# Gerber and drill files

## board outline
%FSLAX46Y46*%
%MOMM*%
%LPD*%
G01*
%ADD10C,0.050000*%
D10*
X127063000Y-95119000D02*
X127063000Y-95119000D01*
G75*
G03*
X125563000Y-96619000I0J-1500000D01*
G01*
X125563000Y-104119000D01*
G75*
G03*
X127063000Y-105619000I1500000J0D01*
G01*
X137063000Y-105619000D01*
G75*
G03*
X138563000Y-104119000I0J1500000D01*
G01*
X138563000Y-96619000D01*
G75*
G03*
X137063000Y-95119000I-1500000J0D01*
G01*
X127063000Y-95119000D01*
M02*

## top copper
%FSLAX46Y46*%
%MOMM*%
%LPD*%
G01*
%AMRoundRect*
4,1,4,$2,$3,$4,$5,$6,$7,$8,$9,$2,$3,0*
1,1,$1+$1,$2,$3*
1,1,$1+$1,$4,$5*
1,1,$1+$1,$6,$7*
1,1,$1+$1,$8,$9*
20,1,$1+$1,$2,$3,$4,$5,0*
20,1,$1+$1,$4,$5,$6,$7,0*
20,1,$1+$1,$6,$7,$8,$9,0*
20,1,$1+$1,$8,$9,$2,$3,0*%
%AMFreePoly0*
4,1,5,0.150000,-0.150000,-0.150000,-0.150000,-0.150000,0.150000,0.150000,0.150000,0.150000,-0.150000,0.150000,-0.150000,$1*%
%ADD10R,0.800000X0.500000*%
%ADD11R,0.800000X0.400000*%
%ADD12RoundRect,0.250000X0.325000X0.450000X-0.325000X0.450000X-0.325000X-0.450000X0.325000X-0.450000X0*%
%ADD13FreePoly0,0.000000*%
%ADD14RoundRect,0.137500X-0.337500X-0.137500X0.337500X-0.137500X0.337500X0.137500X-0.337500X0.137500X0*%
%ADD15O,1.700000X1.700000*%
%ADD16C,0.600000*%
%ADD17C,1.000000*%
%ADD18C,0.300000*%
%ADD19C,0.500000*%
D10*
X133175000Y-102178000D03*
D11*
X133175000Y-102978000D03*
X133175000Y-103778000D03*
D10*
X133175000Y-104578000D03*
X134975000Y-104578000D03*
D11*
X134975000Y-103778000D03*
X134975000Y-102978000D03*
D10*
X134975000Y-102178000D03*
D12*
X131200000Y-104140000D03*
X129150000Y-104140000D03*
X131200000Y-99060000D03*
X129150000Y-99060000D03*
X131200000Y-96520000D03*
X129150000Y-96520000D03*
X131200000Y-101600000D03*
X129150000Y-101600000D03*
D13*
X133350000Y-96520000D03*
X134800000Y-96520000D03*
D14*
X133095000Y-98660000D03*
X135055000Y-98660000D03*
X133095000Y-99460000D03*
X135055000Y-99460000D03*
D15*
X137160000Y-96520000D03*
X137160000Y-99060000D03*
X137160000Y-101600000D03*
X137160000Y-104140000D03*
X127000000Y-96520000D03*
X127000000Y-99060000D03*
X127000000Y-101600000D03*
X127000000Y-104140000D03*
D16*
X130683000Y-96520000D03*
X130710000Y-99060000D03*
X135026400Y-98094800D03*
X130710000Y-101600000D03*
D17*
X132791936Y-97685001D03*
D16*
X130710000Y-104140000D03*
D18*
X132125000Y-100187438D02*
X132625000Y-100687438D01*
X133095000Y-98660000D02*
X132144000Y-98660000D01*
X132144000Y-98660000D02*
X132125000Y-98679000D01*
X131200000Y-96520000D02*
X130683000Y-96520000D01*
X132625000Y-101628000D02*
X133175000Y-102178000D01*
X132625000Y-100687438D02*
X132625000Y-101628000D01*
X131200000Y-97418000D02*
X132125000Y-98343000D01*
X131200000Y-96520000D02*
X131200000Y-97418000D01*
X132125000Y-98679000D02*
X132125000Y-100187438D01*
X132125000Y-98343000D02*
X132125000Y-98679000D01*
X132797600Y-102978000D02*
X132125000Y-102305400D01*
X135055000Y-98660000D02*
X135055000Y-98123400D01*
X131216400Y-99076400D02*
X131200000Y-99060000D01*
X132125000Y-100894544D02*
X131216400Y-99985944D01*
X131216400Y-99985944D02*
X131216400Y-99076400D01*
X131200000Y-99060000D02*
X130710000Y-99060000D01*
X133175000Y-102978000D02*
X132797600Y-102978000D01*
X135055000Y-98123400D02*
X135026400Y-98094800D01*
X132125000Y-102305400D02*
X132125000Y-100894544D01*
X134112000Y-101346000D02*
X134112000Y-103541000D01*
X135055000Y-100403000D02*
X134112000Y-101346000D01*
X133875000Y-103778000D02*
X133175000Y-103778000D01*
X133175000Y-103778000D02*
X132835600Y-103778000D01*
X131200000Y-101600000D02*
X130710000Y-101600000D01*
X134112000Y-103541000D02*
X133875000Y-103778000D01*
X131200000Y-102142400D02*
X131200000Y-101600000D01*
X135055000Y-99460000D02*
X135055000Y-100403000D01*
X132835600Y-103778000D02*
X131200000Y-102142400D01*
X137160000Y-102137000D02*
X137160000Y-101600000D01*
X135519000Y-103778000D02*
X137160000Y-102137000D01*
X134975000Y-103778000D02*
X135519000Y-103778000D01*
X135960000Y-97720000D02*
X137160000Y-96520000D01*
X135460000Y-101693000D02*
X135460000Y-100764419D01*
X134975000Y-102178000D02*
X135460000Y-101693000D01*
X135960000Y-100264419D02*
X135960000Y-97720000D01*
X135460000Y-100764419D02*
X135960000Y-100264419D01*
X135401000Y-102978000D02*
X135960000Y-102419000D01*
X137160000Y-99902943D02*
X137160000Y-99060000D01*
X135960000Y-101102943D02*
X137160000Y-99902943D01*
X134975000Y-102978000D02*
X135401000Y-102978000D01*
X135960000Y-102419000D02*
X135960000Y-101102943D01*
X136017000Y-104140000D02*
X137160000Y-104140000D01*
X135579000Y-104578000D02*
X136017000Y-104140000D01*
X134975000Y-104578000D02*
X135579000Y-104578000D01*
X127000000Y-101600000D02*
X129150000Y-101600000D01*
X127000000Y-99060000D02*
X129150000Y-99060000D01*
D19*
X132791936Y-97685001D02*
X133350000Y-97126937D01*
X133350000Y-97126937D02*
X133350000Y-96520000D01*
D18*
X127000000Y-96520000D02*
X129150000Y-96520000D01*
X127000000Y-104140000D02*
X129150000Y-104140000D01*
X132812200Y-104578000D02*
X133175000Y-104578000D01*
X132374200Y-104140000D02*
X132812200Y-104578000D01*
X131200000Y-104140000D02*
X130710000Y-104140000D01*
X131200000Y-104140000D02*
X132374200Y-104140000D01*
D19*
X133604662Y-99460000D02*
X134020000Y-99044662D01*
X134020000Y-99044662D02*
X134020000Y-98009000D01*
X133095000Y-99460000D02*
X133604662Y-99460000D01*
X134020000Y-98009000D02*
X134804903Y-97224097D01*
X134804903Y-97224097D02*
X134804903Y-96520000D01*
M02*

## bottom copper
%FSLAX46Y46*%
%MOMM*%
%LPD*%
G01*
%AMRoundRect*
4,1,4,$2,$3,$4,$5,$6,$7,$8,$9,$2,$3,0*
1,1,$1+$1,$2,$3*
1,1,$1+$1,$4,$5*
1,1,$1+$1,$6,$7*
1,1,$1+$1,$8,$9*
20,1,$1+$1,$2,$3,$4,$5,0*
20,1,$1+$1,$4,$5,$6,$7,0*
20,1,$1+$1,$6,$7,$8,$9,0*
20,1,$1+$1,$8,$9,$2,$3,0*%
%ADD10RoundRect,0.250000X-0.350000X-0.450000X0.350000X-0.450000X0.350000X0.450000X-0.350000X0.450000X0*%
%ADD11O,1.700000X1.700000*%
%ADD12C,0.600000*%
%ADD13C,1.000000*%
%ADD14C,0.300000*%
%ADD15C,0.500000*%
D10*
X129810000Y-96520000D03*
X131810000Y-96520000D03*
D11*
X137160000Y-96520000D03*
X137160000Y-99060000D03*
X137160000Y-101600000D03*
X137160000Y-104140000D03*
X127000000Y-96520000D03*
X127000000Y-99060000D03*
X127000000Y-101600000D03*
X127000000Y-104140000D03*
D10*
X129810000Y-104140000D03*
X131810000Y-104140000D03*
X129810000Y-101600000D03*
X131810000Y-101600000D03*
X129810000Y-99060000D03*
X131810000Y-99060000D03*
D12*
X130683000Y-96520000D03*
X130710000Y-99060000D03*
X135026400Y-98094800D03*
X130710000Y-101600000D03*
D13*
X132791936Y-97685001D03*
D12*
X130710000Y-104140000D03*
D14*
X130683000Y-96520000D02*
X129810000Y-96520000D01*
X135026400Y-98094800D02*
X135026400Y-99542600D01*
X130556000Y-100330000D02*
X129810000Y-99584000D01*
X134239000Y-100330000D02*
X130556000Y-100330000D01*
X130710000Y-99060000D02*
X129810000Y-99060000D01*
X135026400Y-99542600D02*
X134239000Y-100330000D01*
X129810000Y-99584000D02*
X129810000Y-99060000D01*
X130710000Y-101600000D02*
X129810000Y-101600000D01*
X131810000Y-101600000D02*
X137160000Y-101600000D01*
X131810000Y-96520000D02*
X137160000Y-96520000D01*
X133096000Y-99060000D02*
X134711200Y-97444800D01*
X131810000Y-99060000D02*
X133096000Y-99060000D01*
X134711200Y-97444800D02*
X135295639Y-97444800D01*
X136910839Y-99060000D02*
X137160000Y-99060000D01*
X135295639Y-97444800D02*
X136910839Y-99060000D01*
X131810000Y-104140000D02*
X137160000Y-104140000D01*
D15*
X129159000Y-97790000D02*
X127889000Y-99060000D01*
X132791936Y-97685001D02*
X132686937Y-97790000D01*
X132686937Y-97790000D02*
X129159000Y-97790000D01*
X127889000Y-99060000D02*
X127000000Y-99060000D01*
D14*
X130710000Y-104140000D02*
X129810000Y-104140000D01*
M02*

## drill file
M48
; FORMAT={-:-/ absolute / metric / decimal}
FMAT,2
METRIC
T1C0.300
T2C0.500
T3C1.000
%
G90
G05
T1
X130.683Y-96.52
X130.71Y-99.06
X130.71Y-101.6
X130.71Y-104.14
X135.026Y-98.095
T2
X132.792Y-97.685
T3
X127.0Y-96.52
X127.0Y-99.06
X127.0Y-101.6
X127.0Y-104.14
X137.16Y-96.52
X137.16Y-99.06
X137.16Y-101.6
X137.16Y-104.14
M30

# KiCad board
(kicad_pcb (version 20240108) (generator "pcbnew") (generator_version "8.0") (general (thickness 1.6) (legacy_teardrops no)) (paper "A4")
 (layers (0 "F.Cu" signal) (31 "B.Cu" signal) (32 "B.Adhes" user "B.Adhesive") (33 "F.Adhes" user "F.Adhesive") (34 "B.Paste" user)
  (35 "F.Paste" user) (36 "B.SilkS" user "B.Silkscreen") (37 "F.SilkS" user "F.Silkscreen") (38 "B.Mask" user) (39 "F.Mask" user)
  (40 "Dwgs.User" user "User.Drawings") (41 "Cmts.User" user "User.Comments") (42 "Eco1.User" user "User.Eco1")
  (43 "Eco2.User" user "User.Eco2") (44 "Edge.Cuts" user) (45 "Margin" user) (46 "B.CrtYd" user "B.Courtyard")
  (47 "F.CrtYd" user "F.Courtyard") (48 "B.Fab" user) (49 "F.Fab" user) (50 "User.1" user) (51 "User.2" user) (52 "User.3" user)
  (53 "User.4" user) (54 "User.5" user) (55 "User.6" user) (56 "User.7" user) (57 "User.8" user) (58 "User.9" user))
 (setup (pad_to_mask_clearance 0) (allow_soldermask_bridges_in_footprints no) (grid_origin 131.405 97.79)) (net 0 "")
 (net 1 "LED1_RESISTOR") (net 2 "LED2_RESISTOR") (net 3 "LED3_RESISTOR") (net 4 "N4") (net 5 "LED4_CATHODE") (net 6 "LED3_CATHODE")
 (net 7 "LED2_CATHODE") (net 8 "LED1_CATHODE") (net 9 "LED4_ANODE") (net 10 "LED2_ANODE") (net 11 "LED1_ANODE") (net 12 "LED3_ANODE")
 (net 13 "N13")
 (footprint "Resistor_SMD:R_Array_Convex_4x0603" (layer "F.Cu") (at 134.075 103.378)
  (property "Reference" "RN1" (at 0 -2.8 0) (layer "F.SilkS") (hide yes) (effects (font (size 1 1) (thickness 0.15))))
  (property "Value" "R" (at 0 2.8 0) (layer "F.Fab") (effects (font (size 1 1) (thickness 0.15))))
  (pad "1" smd rect (at -0.9 -1.2) (size 0.8 0.5) (layers "F.Cu" "F.Paste" "F.Mask") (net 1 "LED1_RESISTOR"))
  (pad "2" smd rect (at -0.9 -0.4) (size 0.8 0.4) (layers "F.Cu" "F.Paste" "F.Mask") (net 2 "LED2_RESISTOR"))
  (pad "3" smd rect (at -0.9 0.4) (size 0.8 0.4) (layers "F.Cu" "F.Paste" "F.Mask") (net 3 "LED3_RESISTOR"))
  (pad "4" smd rect (at -0.9 1.2) (size 0.8 0.5) (layers "F.Cu" "F.Paste" "F.Mask") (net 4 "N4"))
  (pad "5" smd rect (at 0.9 1.2) (size 0.8 0.5) (layers "F.Cu" "F.Paste" "F.Mask") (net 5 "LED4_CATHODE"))
  (pad "6" smd rect (at 0.9 0.4) (size 0.8 0.4) (layers "F.Cu" "F.Paste" "F.Mask") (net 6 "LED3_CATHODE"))
  (pad "7" smd rect (at 0.9 -0.4) (size 0.8 0.4) (layers "F.Cu" "F.Paste" "F.Mask") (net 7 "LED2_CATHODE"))
  (pad "8" smd rect (at 0.9 -1.2) (size 0.8 0.5) (layers "F.Cu" "F.Paste" "F.Mask") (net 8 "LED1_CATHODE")))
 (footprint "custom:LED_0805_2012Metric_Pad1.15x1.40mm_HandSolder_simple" (layer "F.Cu") (at 130.175 104.14 180)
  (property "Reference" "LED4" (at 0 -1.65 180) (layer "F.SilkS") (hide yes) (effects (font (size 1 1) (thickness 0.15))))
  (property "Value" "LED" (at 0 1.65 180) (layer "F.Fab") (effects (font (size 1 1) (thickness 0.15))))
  (pad "1" smd roundrect (at -1.025 0 180) (size 1.15 1.4) (layers "F.Cu" "F.Paste" "F.Mask") (roundrect_rratio 0.217391) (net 4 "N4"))
  (pad "2" smd roundrect (at 1.025 0 180) (size 1.15 1.4) (layers "F.Cu" "F.Paste" "F.Mask") (roundrect_rratio 0.217391)
   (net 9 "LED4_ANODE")))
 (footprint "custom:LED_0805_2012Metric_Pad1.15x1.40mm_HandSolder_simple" (layer "F.Cu") (at 130.175 99.06 180)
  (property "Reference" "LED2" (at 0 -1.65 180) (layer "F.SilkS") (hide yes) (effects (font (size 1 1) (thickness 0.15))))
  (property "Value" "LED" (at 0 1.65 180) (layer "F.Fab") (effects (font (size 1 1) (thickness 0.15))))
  (pad "1" smd roundrect (at -1.025 0 180) (size 1.15 1.4) (layers "F.Cu" "F.Paste" "F.Mask") (roundrect_rratio 0.217391)
   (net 2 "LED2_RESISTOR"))
  (pad "2" smd roundrect (at 1.025 0 180) (size 1.15 1.4) (layers "F.Cu" "F.Paste" "F.Mask") (roundrect_rratio 0.217391)
   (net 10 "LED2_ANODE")))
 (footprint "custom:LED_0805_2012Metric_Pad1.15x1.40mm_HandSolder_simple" (layer "F.Cu") (at 130.175 96.52 180)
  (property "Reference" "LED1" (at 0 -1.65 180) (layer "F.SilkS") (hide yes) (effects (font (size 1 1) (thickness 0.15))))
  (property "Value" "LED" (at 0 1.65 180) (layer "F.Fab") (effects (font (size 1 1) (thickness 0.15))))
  (pad "1" smd roundrect (at -1.025 0 180) (size 1.15 1.4) (layers "F.Cu" "F.Paste" "F.Mask") (roundrect_rratio 0.217391)
   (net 1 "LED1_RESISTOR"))
  (pad "2" smd roundrect (at 1.025 0 180) (size 1.15 1.4) (layers "F.Cu" "F.Paste" "F.Mask") (roundrect_rratio 0.217391)
   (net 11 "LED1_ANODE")))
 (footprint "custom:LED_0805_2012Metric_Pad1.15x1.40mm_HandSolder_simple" (layer "F.Cu") (at 130.175 101.6 180)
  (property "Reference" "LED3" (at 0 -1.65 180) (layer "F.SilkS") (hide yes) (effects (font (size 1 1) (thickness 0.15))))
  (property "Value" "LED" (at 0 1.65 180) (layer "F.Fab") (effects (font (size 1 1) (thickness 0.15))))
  (pad "1" smd roundrect (at -1.025 0 180) (size 1.15 1.4) (layers "F.Cu" "F.Paste" "F.Mask") (roundrect_rratio 0.217391)
   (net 3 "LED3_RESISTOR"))
  (pad "2" smd roundrect (at 1.025 0 180) (size 1.15 1.4) (layers "F.Cu" "F.Paste" "F.Mask") (roundrect_rratio 0.217391)
   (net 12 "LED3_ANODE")))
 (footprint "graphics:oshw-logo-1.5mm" (layer "F.Cu") (at 134.874 100.711)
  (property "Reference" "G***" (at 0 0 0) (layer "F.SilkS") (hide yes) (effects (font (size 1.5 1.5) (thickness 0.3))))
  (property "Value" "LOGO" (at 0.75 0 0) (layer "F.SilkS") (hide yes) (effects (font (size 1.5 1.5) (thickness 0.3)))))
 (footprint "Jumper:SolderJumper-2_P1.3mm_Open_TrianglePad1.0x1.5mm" (layer "F.Cu") (at 134.075 96.52)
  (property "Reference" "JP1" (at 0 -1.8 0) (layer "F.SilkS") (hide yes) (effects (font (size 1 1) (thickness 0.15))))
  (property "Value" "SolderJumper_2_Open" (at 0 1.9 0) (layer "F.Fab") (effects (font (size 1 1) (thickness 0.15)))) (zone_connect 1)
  (pad "1" smd custom (at -0.725 0) (size 0.3 0.3) (layers "F.Cu" "F.Mask") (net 10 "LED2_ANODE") (zone_connect 2) (thermal_bridge_angle 45)
   (options (clearance outline) (anchor rect)) (primitives))
  (pad "2" smd custom (at 0.725 0) (size 0.3 0.3) (layers "F.Cu" "F.Mask") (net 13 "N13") (zone_connect 2) (thermal_bridge_angle 45)
   (options (clearance outline) (anchor rect)) (primitives)))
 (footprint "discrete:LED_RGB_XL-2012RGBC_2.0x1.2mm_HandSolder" (layer "F.Cu") (at 134.075 99.06 180)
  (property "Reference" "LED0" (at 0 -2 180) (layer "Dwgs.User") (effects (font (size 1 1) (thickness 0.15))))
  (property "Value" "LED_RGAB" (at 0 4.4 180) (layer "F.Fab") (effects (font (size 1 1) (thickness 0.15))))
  (pad "1" smd roundrect (at 0.98 0.4) (size 0.95 0.55) (layers "F.Cu" "F.Paste" "F.Mask") (roundrect_rratio 0.25) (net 1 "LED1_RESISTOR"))
  (pad "2" smd roundrect (at -0.98 0.4) (size 0.95 0.55) (layers "F.Cu" "F.Paste" "F.Mask") (roundrect_rratio 0.25) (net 2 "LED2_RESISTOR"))
  (pad "3" smd roundrect (at 0.98 -0.4) (size 0.95 0.55) (layers "F.Cu" "F.Paste" "F.Mask") (roundrect_rratio 0.25) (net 13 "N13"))
  (pad "4" smd roundrect (at -0.98 -0.4) (size 0.95 0.55) (layers "F.Cu" "F.Paste" "F.Mask") (roundrect_rratio 0.25) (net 3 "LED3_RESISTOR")))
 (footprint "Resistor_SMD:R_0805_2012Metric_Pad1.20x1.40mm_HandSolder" (layer "B.Cu") (at 130.81 96.52)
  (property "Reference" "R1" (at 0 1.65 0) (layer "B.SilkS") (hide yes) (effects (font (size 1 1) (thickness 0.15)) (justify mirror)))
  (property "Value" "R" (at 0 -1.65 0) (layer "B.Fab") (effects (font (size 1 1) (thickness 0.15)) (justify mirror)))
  (pad "1" smd roundrect (at -1 0) (size 1.2 1.4) (layers "B.Cu" "B.Paste" "B.Mask") (roundrect_rratio 0.208333) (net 1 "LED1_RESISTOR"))
  (pad "2" smd roundrect (at 1 0) (size 1.2 1.4) (layers "B.Cu" "B.Paste" "B.Mask") (roundrect_rratio 0.208333) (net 8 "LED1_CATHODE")))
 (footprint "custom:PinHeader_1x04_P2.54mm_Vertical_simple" (layer "B.Cu") (at 137.16 96.52 180)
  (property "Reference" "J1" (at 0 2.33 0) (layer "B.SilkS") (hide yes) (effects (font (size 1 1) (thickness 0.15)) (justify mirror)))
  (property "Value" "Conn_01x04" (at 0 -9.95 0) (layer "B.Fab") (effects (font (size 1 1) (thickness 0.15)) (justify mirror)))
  (pad "1" thru_hole oval (at 0 0 180) (size 1.7 1.7) (drill 1) (layers "*.Cu" "*.Mask") (remove_unused_layers no) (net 8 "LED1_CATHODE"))
  (pad "2" thru_hole oval (at 0 -2.54 180) (size 1.7 1.7) (drill 1) (layers "*.Cu" "*.Mask") (remove_unused_layers no)
   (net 7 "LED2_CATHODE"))
  (pad "3" thru_hole oval (at 0 -5.08 180) (size 1.7 1.7) (drill 1) (layers "*.Cu" "*.Mask") (remove_unused_layers no)
   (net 6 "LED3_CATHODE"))
  (pad "4" thru_hole oval (at 0 -7.62 180) (size 1.7 1.7) (drill 1) (layers "*.Cu" "*.Mask") (remove_unused_layers no)
   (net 5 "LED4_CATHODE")))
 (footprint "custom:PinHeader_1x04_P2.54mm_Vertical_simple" (layer "B.Cu") (at 127 96.52 180)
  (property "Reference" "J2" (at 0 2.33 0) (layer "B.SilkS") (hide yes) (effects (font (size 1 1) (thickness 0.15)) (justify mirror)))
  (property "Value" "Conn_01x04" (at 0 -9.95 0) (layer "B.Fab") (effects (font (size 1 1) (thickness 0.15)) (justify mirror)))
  (pad "1" thru_hole oval (at 0 0 180) (size 1.7 1.7) (drill 1) (layers "*.Cu" "*.Mask") (remove_unused_layers no) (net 11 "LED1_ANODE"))
  (pad "2" thru_hole oval (at 0 -2.54 180) (size 1.7 1.7) (drill 1) (layers "*.Cu" "*.Mask") (remove_unused_layers no) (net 10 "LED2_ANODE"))
  (pad "3" thru_hole oval (at 0 -5.08 180) (size 1.7 1.7) (drill 1) (layers "*.Cu" "*.Mask") (remove_unused_layers no) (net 12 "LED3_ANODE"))
  (pad "4" thru_hole oval (at 0 -7.62 180) (size 1.7 1.7) (drill 1) (layers "*.Cu" "*.Mask") (remove_unused_layers no) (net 9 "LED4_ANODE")))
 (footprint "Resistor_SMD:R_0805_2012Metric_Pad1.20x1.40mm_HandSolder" (layer "B.Cu") (at 130.81 104.14)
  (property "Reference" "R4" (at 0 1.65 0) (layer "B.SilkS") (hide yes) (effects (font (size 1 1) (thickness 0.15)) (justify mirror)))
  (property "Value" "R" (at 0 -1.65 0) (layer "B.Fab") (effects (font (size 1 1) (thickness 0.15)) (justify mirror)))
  (pad "1" smd roundrect (at -1 0) (size 1.2 1.4) (layers "B.Cu" "B.Paste" "B.Mask") (roundrect_rratio 0.208333) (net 4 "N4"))
  (pad "2" smd roundrect (at 1 0) (size 1.2 1.4) (layers "B.Cu" "B.Paste" "B.Mask") (roundrect_rratio 0.208333) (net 5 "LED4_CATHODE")))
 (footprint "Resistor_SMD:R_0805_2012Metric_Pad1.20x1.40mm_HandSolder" (layer "B.Cu") (at 130.81 101.6)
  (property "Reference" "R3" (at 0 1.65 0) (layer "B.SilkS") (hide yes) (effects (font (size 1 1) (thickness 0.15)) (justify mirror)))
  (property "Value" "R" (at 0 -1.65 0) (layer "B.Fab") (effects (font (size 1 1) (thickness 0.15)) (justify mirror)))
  (pad "1" smd roundrect (at -1 0) (size 1.2 1.4) (layers "B.Cu" "B.Paste" "B.Mask") (roundrect_rratio 0.208333) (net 3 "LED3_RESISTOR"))
  (pad "2" smd roundrect (at 1 0) (size 1.2 1.4) (layers "B.Cu" "B.Paste" "B.Mask") (roundrect_rratio 0.208333) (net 6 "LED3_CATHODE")))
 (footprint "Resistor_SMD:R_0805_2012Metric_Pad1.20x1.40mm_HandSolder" (layer "B.Cu") (at 130.81 99.06)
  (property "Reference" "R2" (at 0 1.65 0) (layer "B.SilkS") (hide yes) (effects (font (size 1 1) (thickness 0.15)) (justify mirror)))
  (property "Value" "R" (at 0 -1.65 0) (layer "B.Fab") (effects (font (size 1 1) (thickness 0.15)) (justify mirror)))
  (pad "1" smd roundrect (at -1 0) (size 1.2 1.4) (layers "B.Cu" "B.Paste" "B.Mask") (roundrect_rratio 0.208333) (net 2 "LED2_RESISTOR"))
  (pad "2" smd roundrect (at 1 0) (size 1.2 1.4) (layers "B.Cu" "B.Paste" "B.Mask") (roundrect_rratio 0.208333) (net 7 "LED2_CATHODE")))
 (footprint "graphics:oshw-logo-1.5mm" (layer "B.Cu") (at 133.55 98.75 90)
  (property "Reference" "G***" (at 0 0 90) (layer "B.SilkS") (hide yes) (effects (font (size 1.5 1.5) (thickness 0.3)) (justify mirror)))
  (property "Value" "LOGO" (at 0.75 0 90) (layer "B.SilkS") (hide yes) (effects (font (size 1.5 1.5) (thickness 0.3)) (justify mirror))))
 (gr_poly
  (pts
   (arc (start 127.063 95.119) (mid 126.00234 95.55834) (end 125.563 96.619))
   (arc (start 125.563 104.119) (mid 126.00234 105.17966) (end 127.063 105.619))
   (arc (start 137.063 105.619) (mid 138.12366 105.17966) (end 138.563 104.119))
   (arc (start 138.563 96.619) (mid 138.12366 95.55834) (end 137.063 95.119)))
  (stroke (width 0.05) (type solid)) (fill none) (layer "Edge.Cuts"))
 (segment (start 132.125 100.187438) (end 132.625 100.687438) (width 0.3) (layer "F.Cu") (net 1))
 (segment (start 133.095 98.66) (end 132.144 98.66) (width 0.3) (layer "F.Cu") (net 1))
 (segment (start 132.144 98.66) (end 132.125 98.679) (width 0.3) (layer "F.Cu") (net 1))
 (segment (start 131.2 96.52) (end 130.683 96.52) (width 0.3) (layer "F.Cu") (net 1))
 (segment (start 132.625 101.628) (end 133.175 102.178) (width 0.3) (layer "F.Cu") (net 1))
 (segment (start 132.625 100.687438) (end 132.625 101.628) (width 0.3) (layer "F.Cu") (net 1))
 (segment (start 131.2 97.418) (end 132.125 98.343) (width 0.3) (layer "F.Cu") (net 1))
 (segment (start 131.2 96.52) (end 131.2 97.418) (width 0.3) (layer "F.Cu") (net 1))
 (segment (start 132.125 98.679) (end 132.125 100.187438) (width 0.3) (layer "F.Cu") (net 1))
 (segment (start 132.125 98.343) (end 132.125 98.679) (width 0.3) (layer "F.Cu") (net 1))
 (via (at 130.683 96.52) (size 0.6) (drill 0.3) (layers "F.Cu" "B.Cu") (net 1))
 (segment (start 130.683 96.52) (end 129.81 96.52) (width 0.3) (layer "B.Cu") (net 1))
 (segment (start 132.7976 102.978) (end 132.125 102.3054) (width 0.3) (layer "F.Cu") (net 2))
 (segment (start 135.055 98.66) (end 135.055 98.1234) (width 0.3) (layer "F.Cu") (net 2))
 (segment (start 131.2164 99.0764) (end 131.2 99.06) (width 0.3) (layer "F.Cu") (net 2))
 (segment (start 132.125 100.894544) (end 131.2164 99.985944) (width 0.3) (layer "F.Cu") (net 2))
 (segment (start 131.2164 99.985944) (end 131.2164 99.0764) (width 0.3) (layer "F.Cu") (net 2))
 (segment (start 131.2 99.06) (end 130.71 99.06) (width 0.3) (layer "F.Cu") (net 2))
 (segment (start 133.175 102.978) (end 132.7976 102.978) (width 0.3) (layer "F.Cu") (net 2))
 (segment (start 135.055 98.1234) (end 135.0264 98.0948) (width 0.3) (layer "F.Cu") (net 2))
 (segment (start 132.125 102.3054) (end 132.125 100.894544) (width 0.3) (layer "F.Cu") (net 2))
 (via (at 130.71 99.06) (size 0.6) (drill 0.3) (layers "F.Cu" "B.Cu") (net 2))
 (via (at 135.0264 98.0948) (size 0.6) (drill 0.3) (layers "F.Cu" "B.Cu") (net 2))
 (segment (start 135.0264 98.0948) (end 135.0264 99.5426) (width 0.3) (layer "B.Cu") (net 2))
 (segment (start 130.556 100.33) (end 129.81 99.584) (width 0.3) (layer "B.Cu") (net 2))
 (segment (start 134.239 100.33) (end 130.556 100.33) (width 0.3) (layer "B.Cu") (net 2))
 (segment (start 130.71 99.06) (end 129.81 99.06) (width 0.3) (layer "B.Cu") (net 2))
 (segment (start 135.0264 99.5426) (end 134.239 100.33) (width 0.3) (layer "B.Cu") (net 2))
 (segment (start 129.81 99.584) (end 129.81 99.06) (width 0.3) (layer "B.Cu") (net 2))
 (segment (start 134.112 101.346) (end 134.112 103.541) (width 0.3) (layer "F.Cu") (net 3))
 (segment (start 135.055 100.403) (end 134.112 101.346) (width 0.3) (layer "F.Cu") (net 3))
 (segment (start 133.875 103.778) (end 133.175 103.778) (width 0.3) (layer "F.Cu") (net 3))
 (segment (start 133.175 103.778) (end 132.8356 103.778) (width 0.3) (layer "F.Cu") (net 3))
 (segment (start 131.2 101.6) (end 130.71 101.6) (width 0.3) (layer "F.Cu") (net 3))
 (segment (start 134.112 103.541) (end 133.875 103.778) (width 0.3) (layer "F.Cu") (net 3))
 (segment (start 131.2 102.1424) (end 131.2 101.6) (width 0.3) (layer "F.Cu") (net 3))
 (segment (start 135.055 99.46) (end 135.055 100.403) (width 0.3) (layer "F.Cu") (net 3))
 (segment (start 132.8356 103.778) (end 131.2 102.1424) (width 0.3) (layer "F.Cu") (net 3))
 (via (at 130.71 101.6) (size 0.6) (drill 0.3) (layers "F.Cu" "B.Cu") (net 3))
 (segment (start 130.71 101.6) (end 129.81 101.6) (width 0.3) (layer "B.Cu") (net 3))
 (segment (start 137.16 102.137) (end 137.16 101.6) (width 0.3) (layer "F.Cu") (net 6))
 (segment (start 135.519 103.778) (end 137.16 102.137) (width 0.3) (layer "F.Cu") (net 6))
 (segment (start 134.975 103.778) (end 135.519 103.778) (width 0.3) (layer "F.Cu") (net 6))
 (segment (start 131.81 101.6) (end 137.16 101.6) (width 0.3) (layer "B.Cu") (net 6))
 (segment (start 135.96 97.72) (end 137.16 96.52) (width 0.3) (layer "F.Cu") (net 8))
 (segment (start 135.46 101.693) (end 135.46 100.764419) (width 0.3) (layer "F.Cu") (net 8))
 (segment (start 134.975 102.178) (end 135.46 101.693) (width 0.3) (layer "F.Cu") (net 8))
 (segment (start 135.96 100.264419) (end 135.96 97.72) (width 0.3) (layer "F.Cu") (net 8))
 (segment (start 135.46 100.764419) (end 135.96 100.264419) (width 0.3) (layer "F.Cu") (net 8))
 (segment (start 131.81 96.52) (end 137.16 96.52) (width 0.3) (layer "B.Cu") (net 8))
 (segment (start 135.401 102.978) (end 135.96 102.419) (width 0.3) (layer "F.Cu") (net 7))
 (segment (start 137.16 99.902943) (end 137.16 99.06) (width 0.3) (layer "F.Cu") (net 7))
 (segment (start 135.96 101.102943) (end 137.16 99.902943) (width 0.3) (layer "F.Cu") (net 7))
 (segment (start 134.975 102.978) (end 135.401 102.978) (width 0.3) (layer "F.Cu") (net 7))
 (segment (start 135.96 102.419) (end 135.96 101.102943) (width 0.3) (layer "F.Cu") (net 7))
 (segment (start 133.096 99.06) (end 134.7112 97.4448) (width 0.3) (layer "B.Cu") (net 7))
 (segment (start 131.81 99.06) (end 133.096 99.06) (width 0.3) (layer "B.Cu") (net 7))
 (segment (start 134.7112 97.4448) (end 135.295639 97.4448) (width 0.3) (layer "B.Cu") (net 7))
 (segment (start 136.910839 99.06) (end 137.16 99.06) (width 0.3) (layer "B.Cu") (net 7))
 (segment (start 135.295639 97.4448) (end 136.910839 99.06) (width 0.3) (layer "B.Cu") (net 7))
 (segment (start 136.017 104.14) (end 137.16 104.14) (width 0.3) (layer "F.Cu") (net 5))
 (segment (start 135.579 104.578) (end 136.017 104.14) (width 0.3) (layer "F.Cu") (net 5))
 (segment (start 134.975 104.578) (end 135.579 104.578) (width 0.3) (layer "F.Cu") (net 5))
 (segment (start 131.81 104.14) (end 137.16 104.14) (width 0.3) (layer "B.Cu") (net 5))
 (segment (start 127 101.6) (end 129.15 101.6) (width 0.3) (layer "F.Cu") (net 12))
 (segment (start 127 99.06) (end 129.15 99.06) (width 0.3) (layer "F.Cu") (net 10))
 (segment (start 132.791936 97.685001) (end 133.35 97.126937) (width 0.5) (layer "F.Cu") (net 10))
 (segment (start 133.35 97.126937) (end 133.35 96.52) (width 0.5) (layer "F.Cu") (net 10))
 (via (at 132.791936 97.685001) (size 1) (drill 0.5) (layers "F.Cu" "B.Cu") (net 10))
 (segment (start 129.159 97.79) (end 127.889 99.06) (width 0.5) (layer "B.Cu") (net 10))
 (segment (start 132.791936 97.685001) (end 132.686937 97.79) (width 0.5) (layer "B.Cu") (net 10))
 (segment (start 132.686937 97.79) (end 129.159 97.79) (width 0.5) (layer "B.Cu") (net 10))
 (segment (start 127.889 99.06) (end 127 99.06) (width 0.5) (layer "B.Cu") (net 10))
 (segment (start 127 96.52) (end 129.15 96.52) (width 0.3) (layer "F.Cu") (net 11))
 (segment (start 127 104.14) (end 129.15 104.14) (width 0.3) (layer "F.Cu") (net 9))
 (segment (start 132.8122 104.578) (end 133.175 104.578) (width 0.3) (layer "F.Cu") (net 4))
 (segment (start 132.3742 104.14) (end 132.8122 104.578) (width 0.3) (layer "F.Cu") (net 4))
 (segment (start 131.2 104.14) (end 130.71 104.14) (width 0.3) (layer "F.Cu") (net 4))
 (segment (start 131.2 104.14) (end 132.3742 104.14) (width 0.3) (layer "F.Cu") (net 4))
 (via (at 130.71 104.14) (size 0.6) (drill 0.3) (layers "F.Cu" "B.Cu") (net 4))
 (segment (start 130.71 104.14) (end 129.81 104.14) (width 0.3) (layer "B.Cu") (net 4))
 (segment (start 133.604662 99.46) (end 134.02 99.044662) (width 0.5) (layer "F.Cu") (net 13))
 (segment (start 134.02 99.044662) (end 134.02 98.009) (width 0.5) (layer "F.Cu") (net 13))
 (segment (start 133.095 99.46) (end 133.604662 99.46) (width 0.5) (layer "F.Cu") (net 13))
 (segment (start 134.02 98.009) (end 134.804903 97.224097) (width 0.5) (layer "F.Cu") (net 13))
 (segment (start 134.804903 97.224097) (end 134.804903 96.52) (width 0.5) (layer "F.Cu") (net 13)))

